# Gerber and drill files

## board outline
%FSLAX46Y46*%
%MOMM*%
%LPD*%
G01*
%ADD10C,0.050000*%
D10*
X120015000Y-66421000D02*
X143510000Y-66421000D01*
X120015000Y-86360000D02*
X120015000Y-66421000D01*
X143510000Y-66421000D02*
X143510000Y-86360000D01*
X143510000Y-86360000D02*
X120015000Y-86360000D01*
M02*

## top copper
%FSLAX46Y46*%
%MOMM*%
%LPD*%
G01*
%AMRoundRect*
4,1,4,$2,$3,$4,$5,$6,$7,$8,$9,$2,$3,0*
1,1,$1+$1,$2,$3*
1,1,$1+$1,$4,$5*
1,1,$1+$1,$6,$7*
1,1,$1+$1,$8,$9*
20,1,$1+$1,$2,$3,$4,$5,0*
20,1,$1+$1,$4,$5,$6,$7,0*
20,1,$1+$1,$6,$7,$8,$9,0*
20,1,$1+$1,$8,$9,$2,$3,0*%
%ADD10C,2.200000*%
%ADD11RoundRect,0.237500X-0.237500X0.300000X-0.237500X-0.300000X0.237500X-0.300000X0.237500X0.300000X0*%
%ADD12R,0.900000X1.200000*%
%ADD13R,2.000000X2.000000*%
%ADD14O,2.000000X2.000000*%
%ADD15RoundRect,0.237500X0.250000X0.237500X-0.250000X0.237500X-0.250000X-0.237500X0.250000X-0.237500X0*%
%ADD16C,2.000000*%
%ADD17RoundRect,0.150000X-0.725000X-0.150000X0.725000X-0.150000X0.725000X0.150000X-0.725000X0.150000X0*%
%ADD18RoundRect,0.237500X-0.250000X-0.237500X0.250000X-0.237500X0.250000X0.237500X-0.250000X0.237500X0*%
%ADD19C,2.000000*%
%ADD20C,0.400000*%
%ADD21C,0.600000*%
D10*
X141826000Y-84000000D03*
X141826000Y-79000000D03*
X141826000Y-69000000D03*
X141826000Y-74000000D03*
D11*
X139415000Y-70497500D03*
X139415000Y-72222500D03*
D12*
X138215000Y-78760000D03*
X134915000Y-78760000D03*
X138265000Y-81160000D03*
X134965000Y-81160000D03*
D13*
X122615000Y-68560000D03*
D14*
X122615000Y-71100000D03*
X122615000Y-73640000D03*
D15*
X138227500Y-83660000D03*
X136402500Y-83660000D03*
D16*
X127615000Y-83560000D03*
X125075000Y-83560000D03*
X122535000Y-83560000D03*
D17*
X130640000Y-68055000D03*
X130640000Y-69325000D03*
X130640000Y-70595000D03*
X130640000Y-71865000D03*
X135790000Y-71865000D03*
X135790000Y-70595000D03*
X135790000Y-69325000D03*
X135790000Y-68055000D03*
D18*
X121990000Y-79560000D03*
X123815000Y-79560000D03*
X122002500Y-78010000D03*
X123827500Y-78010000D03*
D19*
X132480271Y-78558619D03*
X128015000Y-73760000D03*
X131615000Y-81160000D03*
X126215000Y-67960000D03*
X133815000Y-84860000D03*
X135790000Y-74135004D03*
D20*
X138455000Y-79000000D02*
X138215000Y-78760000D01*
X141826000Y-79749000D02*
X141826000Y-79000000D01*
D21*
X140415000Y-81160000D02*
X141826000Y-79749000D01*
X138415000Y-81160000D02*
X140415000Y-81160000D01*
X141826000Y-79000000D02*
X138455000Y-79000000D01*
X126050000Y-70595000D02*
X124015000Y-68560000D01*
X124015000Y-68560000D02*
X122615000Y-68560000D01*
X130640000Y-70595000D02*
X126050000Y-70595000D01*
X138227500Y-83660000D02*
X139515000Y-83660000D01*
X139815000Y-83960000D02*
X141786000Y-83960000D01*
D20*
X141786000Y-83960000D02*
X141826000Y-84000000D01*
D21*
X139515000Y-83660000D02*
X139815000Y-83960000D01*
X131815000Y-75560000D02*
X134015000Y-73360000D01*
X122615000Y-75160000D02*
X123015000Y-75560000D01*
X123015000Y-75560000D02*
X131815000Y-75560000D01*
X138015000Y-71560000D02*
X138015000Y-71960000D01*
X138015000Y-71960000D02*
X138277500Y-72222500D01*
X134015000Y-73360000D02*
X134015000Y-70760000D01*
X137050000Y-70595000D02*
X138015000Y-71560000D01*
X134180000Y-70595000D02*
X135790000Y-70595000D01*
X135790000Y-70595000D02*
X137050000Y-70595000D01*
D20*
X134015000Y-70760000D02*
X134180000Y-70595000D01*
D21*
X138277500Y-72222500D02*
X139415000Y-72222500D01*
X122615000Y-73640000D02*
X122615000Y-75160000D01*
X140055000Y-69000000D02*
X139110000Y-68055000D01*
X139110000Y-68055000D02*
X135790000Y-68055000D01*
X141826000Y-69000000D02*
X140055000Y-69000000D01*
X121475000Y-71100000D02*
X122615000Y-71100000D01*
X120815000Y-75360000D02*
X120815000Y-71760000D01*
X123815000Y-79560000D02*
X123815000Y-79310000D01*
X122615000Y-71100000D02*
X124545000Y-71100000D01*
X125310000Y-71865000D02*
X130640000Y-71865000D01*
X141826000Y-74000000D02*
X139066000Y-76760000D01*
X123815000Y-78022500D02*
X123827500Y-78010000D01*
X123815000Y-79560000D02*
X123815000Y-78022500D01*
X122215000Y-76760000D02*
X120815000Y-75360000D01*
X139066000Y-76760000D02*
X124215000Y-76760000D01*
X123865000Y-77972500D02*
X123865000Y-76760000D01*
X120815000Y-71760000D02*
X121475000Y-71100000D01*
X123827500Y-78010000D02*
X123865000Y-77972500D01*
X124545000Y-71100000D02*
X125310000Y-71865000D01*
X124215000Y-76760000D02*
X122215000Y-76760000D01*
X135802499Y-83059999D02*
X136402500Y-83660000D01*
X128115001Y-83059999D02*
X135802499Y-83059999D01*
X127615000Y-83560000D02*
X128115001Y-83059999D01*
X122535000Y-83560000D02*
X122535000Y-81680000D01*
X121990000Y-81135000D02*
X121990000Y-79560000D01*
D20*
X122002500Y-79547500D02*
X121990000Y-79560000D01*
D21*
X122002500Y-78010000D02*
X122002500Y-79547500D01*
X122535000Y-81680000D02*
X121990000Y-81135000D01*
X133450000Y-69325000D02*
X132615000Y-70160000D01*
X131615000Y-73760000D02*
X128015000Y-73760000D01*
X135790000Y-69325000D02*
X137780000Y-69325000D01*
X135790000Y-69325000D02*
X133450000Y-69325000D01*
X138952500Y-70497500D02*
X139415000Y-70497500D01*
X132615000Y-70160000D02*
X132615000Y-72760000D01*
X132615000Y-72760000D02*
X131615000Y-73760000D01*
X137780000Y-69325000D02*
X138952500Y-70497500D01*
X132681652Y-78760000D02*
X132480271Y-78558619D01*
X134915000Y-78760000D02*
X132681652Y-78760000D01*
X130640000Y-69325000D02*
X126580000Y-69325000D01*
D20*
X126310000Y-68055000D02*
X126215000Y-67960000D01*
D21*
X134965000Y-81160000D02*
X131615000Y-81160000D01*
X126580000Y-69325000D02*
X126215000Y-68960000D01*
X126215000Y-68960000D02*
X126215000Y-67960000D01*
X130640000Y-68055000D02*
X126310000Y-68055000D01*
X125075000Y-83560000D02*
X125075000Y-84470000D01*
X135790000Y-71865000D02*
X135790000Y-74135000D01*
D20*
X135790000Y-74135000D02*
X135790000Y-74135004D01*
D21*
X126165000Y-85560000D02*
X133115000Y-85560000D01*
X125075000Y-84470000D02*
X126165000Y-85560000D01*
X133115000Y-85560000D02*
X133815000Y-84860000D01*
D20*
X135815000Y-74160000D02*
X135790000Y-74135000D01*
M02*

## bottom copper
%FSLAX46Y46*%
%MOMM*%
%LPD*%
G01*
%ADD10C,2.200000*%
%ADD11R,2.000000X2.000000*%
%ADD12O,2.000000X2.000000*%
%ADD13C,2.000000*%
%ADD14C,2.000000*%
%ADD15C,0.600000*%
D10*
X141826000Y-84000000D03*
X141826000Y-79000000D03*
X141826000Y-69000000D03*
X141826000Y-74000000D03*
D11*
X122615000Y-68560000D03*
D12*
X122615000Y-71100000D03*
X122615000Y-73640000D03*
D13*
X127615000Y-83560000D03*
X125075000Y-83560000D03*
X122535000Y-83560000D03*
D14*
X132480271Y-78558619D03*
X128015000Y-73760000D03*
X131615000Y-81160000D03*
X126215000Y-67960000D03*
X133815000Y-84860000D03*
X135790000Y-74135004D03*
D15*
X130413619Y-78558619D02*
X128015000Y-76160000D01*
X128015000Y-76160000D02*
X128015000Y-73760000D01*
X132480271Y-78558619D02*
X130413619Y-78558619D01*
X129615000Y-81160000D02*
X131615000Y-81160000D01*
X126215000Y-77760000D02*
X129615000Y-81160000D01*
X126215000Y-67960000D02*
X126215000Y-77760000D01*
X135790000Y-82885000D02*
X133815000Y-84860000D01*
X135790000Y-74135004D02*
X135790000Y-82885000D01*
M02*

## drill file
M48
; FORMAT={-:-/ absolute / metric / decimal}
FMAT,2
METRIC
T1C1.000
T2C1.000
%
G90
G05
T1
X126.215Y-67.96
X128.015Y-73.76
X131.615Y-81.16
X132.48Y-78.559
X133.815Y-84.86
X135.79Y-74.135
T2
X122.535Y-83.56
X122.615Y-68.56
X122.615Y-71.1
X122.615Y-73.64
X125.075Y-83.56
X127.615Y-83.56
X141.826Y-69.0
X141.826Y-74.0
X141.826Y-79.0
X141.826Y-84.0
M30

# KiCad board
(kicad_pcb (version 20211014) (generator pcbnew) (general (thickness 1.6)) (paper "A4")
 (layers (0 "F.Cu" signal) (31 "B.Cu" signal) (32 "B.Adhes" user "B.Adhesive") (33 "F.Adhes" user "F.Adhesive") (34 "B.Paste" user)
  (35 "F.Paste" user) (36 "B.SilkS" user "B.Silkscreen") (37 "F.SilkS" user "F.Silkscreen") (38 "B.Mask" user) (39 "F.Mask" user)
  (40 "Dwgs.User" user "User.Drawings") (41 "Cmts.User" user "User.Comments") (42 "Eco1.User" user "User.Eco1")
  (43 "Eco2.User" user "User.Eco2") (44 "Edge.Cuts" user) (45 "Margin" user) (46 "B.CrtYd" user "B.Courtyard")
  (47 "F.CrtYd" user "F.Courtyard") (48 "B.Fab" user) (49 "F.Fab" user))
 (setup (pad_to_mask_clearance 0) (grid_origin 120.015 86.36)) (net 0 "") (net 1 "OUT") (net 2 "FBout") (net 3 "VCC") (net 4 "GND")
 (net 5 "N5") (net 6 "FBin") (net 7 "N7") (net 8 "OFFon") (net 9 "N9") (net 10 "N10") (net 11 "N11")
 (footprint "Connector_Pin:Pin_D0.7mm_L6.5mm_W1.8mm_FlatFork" (layer "F.Cu") (at 141.826 84)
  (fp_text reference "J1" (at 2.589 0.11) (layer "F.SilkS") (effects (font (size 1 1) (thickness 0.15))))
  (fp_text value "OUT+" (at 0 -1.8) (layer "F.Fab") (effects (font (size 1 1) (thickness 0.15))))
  (pad "1" thru_hole circle locked (at 0 0) (size 2.2 2.2) (drill 1) (layers *.Cu *.Mask) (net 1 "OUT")))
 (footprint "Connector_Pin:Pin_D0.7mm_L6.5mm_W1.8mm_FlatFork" (layer "F.Cu") (at 141.826 79)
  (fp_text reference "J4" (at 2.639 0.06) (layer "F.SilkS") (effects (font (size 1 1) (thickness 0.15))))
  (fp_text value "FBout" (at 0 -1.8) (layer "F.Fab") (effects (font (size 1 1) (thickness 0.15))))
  (pad "1" thru_hole circle locked (at 0 0) (size 2.2 2.2) (drill 1) (layers *.Cu *.Mask) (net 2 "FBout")))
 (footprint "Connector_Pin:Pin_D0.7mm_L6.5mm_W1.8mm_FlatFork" (layer "F.Cu") (at 141.826 69)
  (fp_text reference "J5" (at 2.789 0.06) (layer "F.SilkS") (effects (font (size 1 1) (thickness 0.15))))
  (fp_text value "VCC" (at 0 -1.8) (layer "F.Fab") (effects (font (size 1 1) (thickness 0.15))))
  (pad "1" thru_hole circle locked (at 0 0) (size 2.2 2.2) (drill 1) (layers *.Cu *.Mask) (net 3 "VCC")))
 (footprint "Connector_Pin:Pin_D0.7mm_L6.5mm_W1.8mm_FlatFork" (layer "F.Cu") (at 141.826 74)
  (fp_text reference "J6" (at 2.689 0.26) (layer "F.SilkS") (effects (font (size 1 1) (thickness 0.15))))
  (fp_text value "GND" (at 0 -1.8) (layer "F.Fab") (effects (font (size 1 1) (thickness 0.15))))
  (pad "1" thru_hole circle locked (at 0 0) (size 2.2 2.2) (drill 1) (layers *.Cu *.Mask) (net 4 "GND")))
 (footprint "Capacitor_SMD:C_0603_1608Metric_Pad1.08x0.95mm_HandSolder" (layer "F.Cu") (at 139.415 71.36 -90)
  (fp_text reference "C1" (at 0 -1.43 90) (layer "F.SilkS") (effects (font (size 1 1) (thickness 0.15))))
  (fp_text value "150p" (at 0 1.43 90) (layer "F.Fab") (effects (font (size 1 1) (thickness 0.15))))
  (pad "1" smd roundrect locked (at -0.8625 0 270) (size 1.075 0.95) (layers "F.Cu" "F.Paste" "F.Mask") (roundrect_rratio 0.25) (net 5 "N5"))
  (pad "2" smd roundrect locked (at 0.8625 0 270) (size 1.075 0.95) (layers "F.Cu" "F.Paste" "F.Mask") (roundrect_rratio 0.25)
   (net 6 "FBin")))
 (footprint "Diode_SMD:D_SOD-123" (layer "F.Cu") (at 136.565 78.76 180)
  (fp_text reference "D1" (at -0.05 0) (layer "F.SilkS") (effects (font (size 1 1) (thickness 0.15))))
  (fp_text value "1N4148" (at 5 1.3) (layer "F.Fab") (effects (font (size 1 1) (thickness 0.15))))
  (pad "1" smd rect locked (at -1.65 0 180) (size 0.9 1.2) (layers "F.Cu" "F.Paste" "F.Mask") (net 2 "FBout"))
  (pad "2" smd rect locked (at 1.65 0 180) (size 0.9 1.2) (layers "F.Cu" "F.Paste" "F.Mask") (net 5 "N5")))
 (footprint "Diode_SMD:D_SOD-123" (layer "F.Cu") (at 136.615 81.16 180)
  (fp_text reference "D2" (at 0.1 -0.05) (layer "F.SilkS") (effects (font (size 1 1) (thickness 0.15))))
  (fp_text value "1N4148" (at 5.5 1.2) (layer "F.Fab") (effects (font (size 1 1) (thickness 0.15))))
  (pad "1" smd rect locked (at -1.65 0 180) (size 0.9 1.2) (layers "F.Cu" "F.Paste" "F.Mask") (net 2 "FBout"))
  (pad "2" smd rect locked (at 1.65 0 180) (size 0.9 1.2) (layers "F.Cu" "F.Paste" "F.Mask") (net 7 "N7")))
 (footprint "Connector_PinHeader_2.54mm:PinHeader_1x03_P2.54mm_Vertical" (layer "F.Cu") (at 122.615 68.56)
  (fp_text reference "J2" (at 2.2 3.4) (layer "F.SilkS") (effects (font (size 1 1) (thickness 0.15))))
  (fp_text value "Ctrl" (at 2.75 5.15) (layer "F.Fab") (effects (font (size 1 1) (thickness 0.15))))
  (pad "1" thru_hole rect locked (at 0 0) (size 2 2) (drill 1) (layers *.Cu *.Mask) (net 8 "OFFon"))
  (pad "2" thru_hole oval locked (at 0 2.54) (size 2 2) (drill 1) (layers *.Cu *.Mask) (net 4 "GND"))
  (pad "3" thru_hole oval locked (at 0 5.08) (size 2 2) (drill 1) (layers *.Cu *.Mask) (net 6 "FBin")))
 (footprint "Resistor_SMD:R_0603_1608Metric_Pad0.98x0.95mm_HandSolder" (layer "F.Cu") (at 137.315 83.66 180)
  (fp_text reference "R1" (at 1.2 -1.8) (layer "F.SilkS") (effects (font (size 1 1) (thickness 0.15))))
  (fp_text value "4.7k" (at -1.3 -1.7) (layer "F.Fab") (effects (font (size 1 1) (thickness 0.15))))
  (pad "1" smd roundrect locked (at -0.9125 0 180) (size 0.975 0.95) (layers "F.Cu" "F.Paste" "F.Mask") (roundrect_rratio 0.25)
   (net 1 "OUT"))
  (pad "2" smd roundrect locked (at 0.9125 0 180) (size 0.975 0.95) (layers "F.Cu" "F.Paste" "F.Mask") (roundrect_rratio 0.25) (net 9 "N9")))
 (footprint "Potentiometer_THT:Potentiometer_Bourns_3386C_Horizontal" (layer "F.Cu") (at 127.615 83.56 -90)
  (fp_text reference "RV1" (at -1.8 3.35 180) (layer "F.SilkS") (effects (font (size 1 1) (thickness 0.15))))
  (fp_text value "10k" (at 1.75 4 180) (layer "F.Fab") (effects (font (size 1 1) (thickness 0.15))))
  (pad "1" thru_hole circle locked (at 0 0 270) (size 2 2) (drill 1) (layers *.Cu *.Mask) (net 9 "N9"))
  (pad "2" thru_hole circle locked (at 0 2.54 270) (size 2 2) (drill 1) (layers *.Cu *.Mask) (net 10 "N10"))
  (pad "3" thru_hole circle locked (at 0 5.08 270) (size 2 2) (drill 1) (layers *.Cu *.Mask) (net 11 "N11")))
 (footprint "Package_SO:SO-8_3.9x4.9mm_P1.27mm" (layer "F.Cu") (at 133.215 69.96)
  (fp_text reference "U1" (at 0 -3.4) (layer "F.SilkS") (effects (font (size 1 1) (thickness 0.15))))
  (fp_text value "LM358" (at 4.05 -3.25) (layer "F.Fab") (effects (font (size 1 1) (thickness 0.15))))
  (pad "1" smd roundrect locked (at -2.575 -1.905) (size 1.75 0.6) (layers "F.Cu" "F.Paste" "F.Mask") (roundrect_rratio 0.25) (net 7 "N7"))
  (pad "2" smd roundrect locked (at -2.575 -0.635) (size 1.75 0.6) (layers "F.Cu" "F.Paste" "F.Mask") (roundrect_rratio 0.25) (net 7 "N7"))
  (pad "3" smd roundrect locked (at -2.575 0.635) (size 1.75 0.6) (layers "F.Cu" "F.Paste" "F.Mask") (roundrect_rratio 0.25) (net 8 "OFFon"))
  (pad "4" smd roundrect locked (at -2.575 1.905) (size 1.75 0.6) (layers "F.Cu" "F.Paste" "F.Mask") (roundrect_rratio 0.25) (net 4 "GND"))
  (pad "5" smd roundrect locked (at 2.575 1.905) (size 1.75 0.6) (layers "F.Cu" "F.Paste" "F.Mask") (roundrect_rratio 0.25) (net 10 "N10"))
  (pad "6" smd roundrect locked (at 2.575 0.635) (size 1.75 0.6) (layers "F.Cu" "F.Paste" "F.Mask") (roundrect_rratio 0.25) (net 6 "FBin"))
  (pad "7" smd roundrect locked (at 2.575 -0.635) (size 1.75 0.6) (layers "F.Cu" "F.Paste" "F.Mask") (roundrect_rratio 0.25) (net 5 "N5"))
  (pad "8" smd roundrect locked (at 2.575 -1.905) (size 1.75 0.6) (layers "F.Cu" "F.Paste" "F.Mask") (roundrect_rratio 0.25) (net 3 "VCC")))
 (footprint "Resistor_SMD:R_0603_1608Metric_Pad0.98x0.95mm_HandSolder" (layer "F.Cu") (at 122.9025 79.56)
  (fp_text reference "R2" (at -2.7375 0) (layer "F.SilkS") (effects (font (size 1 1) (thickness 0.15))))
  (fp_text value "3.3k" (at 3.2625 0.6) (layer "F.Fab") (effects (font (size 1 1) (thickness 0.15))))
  (pad "1" smd roundrect locked (at -0.9125 0) (size 0.975 0.95) (layers "F.Cu" "F.Paste" "F.Mask") (roundrect_rratio 0.25) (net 11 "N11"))
  (pad "2" smd roundrect locked (at 0.9125 0) (size 0.975 0.95) (layers "F.Cu" "F.Paste" "F.Mask") (roundrect_rratio 0.25) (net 4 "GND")))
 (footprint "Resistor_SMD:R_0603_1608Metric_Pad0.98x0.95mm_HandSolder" (layer "F.Cu") (at 122.915 78.01)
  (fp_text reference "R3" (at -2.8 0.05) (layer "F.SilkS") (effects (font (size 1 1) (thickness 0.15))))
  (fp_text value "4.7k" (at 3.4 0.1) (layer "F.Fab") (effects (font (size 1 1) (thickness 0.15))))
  (pad "1" smd roundrect locked (at -0.9125 0) (size 0.975 0.95) (layers "F.Cu" "F.Paste" "F.Mask") (roundrect_rratio 0.25) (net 11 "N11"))
  (pad "2" smd roundrect locked (at 0.9125 0) (size 0.975 0.95) (layers "F.Cu" "F.Paste" "F.Mask") (roundrect_rratio 0.25) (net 4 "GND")))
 (gr_line (start 120.015 66.421) (end 143.51 66.421) (layer "Edge.Cuts") (width 0.05))
 (gr_line (start 120.015 86.36) (end 120.015 66.421) (layer "Edge.Cuts") (width 0.05))
 (gr_line (start 143.51 66.421) (end 143.51 86.36) (layer "Edge.Cuts") (width 0.05))
 (gr_line (start 143.51 86.36) (end 120.015 86.36) (layer "Edge.Cuts") (width 0.05))
 (segment (start 138.455 79) (end 138.215 78.76) (width 0.4) (layer "F.Cu") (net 2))
 (segment (start 141.826 79.749) (end 141.826 79) (width 0.4) (layer "F.Cu") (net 2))
 (segment (start 140.415 81.16) (end 141.826 79.749) (width 0.6) (layer "F.Cu") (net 2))
 (segment (start 138.415 81.16) (end 140.415 81.16) (width 0.6) (layer "F.Cu") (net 2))
 (segment (start 141.826 79) (end 138.455 79) (width 0.6) (layer "F.Cu") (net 2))
 (segment (start 126.05 70.595) (end 124.015 68.56) (width 0.6) (layer "F.Cu") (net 8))
 (segment (start 124.015 68.56) (end 122.615 68.56) (width 0.6) (layer "F.Cu") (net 8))
 (segment (start 130.64 70.595) (end 126.05 70.595) (width 0.6) (layer "F.Cu") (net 8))
 (segment (start 138.2275 83.66) (end 139.515 83.66) (width 0.6) (layer "F.Cu") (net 1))
 (segment (start 139.815 83.96) (end 141.786 83.96) (width 0.6) (layer "F.Cu") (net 1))
 (segment (start 141.786 83.96) (end 141.826 84) (width 0.4) (layer "F.Cu") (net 1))
 (segment (start 139.515 83.66) (end 139.815 83.96) (width 0.6) (layer "F.Cu") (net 1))
 (segment (start 131.815 75.56) (end 134.015 73.36) (width 0.6) (layer "F.Cu") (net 6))
 (segment (start 122.615 75.16) (end 123.015 75.56) (width 0.6) (layer "F.Cu") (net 6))
 (segment (start 123.015 75.56) (end 131.815 75.56) (width 0.6) (layer "F.Cu") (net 6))
 (segment (start 138.015 71.56) (end 138.015 71.96) (width 0.6) (layer "F.Cu") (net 6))
 (segment (start 138.015 71.96) (end 138.2775 72.2225) (width 0.6) (layer "F.Cu") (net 6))
 (segment (start 134.015 73.36) (end 134.015 70.76) (width 0.6) (layer "F.Cu") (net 6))
 (segment (start 137.05 70.595) (end 138.015 71.56) (width 0.6) (layer "F.Cu") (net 6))
 (segment (start 134.18 70.595) (end 135.79 70.595) (width 0.6) (layer "F.Cu") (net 6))
 (segment (start 135.79 70.595) (end 137.05 70.595) (width 0.6) (layer "F.Cu") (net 6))
 (segment (start 134.015 70.76) (end 134.18 70.595) (width 0.4) (layer "F.Cu") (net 6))
 (segment (start 138.2775 72.2225) (end 139.415 72.2225) (width 0.6) (layer "F.Cu") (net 6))
 (segment (start 122.615 73.64) (end 122.615 75.16) (width 0.6) (layer "F.Cu") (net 6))
 (segment (start 140.055 69) (end 139.11 68.055) (width 0.6) (layer "F.Cu") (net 3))
 (segment (start 139.11 68.055) (end 135.79 68.055) (width 0.6) (layer "F.Cu") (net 3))
 (segment (start 141.826 69) (end 140.055 69) (width 0.6) (layer "F.Cu") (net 3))
 (segment (start 121.475 71.1) (end 122.615 71.1) (width 0.6) (layer "F.Cu") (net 4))
 (segment (start 120.815 75.36) (end 120.815 71.76) (width 0.6) (layer "F.Cu") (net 4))
 (segment (start 123.815 79.56) (end 123.815 79.31) (width 0.6) (layer "F.Cu") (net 4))
 (segment (start 122.615 71.1) (end 124.545 71.1) (width 0.6) (layer "F.Cu") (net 4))
 (segment (start 125.31 71.865) (end 130.64 71.865) (width 0.6) (layer "F.Cu") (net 4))
 (segment (start 141.826 74) (end 139.066 76.76) (width 0.6) (layer "F.Cu") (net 4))
 (segment (start 123.815 78.0225) (end 123.8275 78.01) (width 0.6) (layer "F.Cu") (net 4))
 (segment (start 123.815 79.56) (end 123.815 78.0225) (width 0.6) (layer "F.Cu") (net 4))
 (segment (start 122.215 76.76) (end 120.815 75.36) (width 0.6) (layer "F.Cu") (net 4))
 (segment (start 139.066 76.76) (end 124.215 76.76) (width 0.6) (layer "F.Cu") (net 4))
 (segment (start 123.865 77.9725) (end 123.865 76.76) (width 0.6) (layer "F.Cu") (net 4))
 (segment (start 120.815 71.76) (end 121.475 71.1) (width 0.6) (layer "F.Cu") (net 4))
 (segment (start 123.8275 78.01) (end 123.865 77.9725) (width 0.6) (layer "F.Cu") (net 4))
 (segment (start 124.545 71.1) (end 125.31 71.865) (width 0.6) (layer "F.Cu") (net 4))
 (segment (start 124.215 76.76) (end 122.215 76.76) (width 0.6) (layer "F.Cu") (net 4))
 (segment (start 135.802499 83.059999) (end 136.4025 83.66) (width 0.6) (layer "F.Cu") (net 9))
 (segment (start 128.115001 83.059999) (end 135.802499 83.059999) (width 0.6) (layer "F.Cu") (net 9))
 (segment (start 127.615 83.56) (end 128.115001 83.059999) (width 0.6) (layer "F.Cu") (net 9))
 (segment (start 122.535 83.56) (end 122.535 81.68) (width 0.6) (layer "F.Cu") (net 11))
 (segment (start 121.99 81.135) (end 121.99 79.56) (width 0.6) (layer "F.Cu") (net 11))
 (segment (start 122.0025 79.5475) (end 121.99 79.56) (width 0.4) (layer "F.Cu") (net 11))
 (segment (start 122.0025 78.01) (end 122.0025 79.5475) (width 0.6) (layer "F.Cu") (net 11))
 (segment (start 122.535 81.68) (end 121.99 81.135) (width 0.6) (layer "F.Cu") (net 11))
 (segment (start 133.45 69.325) (end 132.615 70.16) (width 0.6) (layer "F.Cu") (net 5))
 (segment (start 131.615 73.76) (end 128.015 73.76) (width 0.6) (layer "F.Cu") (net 5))
 (segment (start 135.79 69.325) (end 137.78 69.325) (width 0.6) (layer "F.Cu") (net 5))
 (segment (start 135.79 69.325) (end 133.45 69.325) (width 0.6) (layer "F.Cu") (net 5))
 (segment (start 138.9525 70.4975) (end 139.415 70.4975) (width 0.6) (layer "F.Cu") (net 5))
 (segment (start 132.615 70.16) (end 132.615 72.76) (width 0.6) (layer "F.Cu") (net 5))
 (segment (start 132.615 72.76) (end 131.615 73.76) (width 0.6) (layer "F.Cu") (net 5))
 (segment (start 137.78 69.325) (end 138.9525 70.4975) (width 0.6) (layer "F.Cu") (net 5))
 (segment (start 132.681652 78.76) (end 132.480271 78.558619) (width 0.6) (layer "F.Cu") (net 5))
 (segment (start 134.915 78.76) (end 132.681652 78.76) (width 0.6) (layer "F.Cu") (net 5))
 (via (at 132.480271 78.558619) (size 2) (drill 1) (layers "F.Cu" "B.Cu") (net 5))
 (via (at 128.015 73.76) (size 2) (drill 1) (layers "F.Cu" "B.Cu") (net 5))
 (segment (start 130.413619 78.558619) (end 128.015 76.16) (width 0.6) (layer "B.Cu") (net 5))
 (segment (start 128.015 76.16) (end 128.015 73.76) (width 0.6) (layer "B.Cu") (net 5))
 (segment (start 132.480271 78.558619) (end 130.413619 78.558619) (width 0.6) (layer "B.Cu") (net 5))
 (segment (start 130.64 69.325) (end 126.58 69.325) (width 0.6) (layer "F.Cu") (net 7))
 (segment (start 126.31 68.055) (end 126.215 67.96) (width 0.4) (layer "F.Cu") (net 7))
 (segment (start 134.965 81.16) (end 131.615 81.16) (width 0.6) (layer "F.Cu") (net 7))
 (segment (start 126.58 69.325) (end 126.215 68.96) (width 0.6) (layer "F.Cu") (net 7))
 (segment (start 126.215 68.96) (end 126.215 67.96) (width 0.6) (layer "F.Cu") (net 7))
 (segment (start 130.64 68.055) (end 126.31 68.055) (width 0.6) (layer "F.Cu") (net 7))
 (via (at 131.615 81.16) (size 2) (drill 1) (layers "F.Cu" "B.Cu") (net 7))
 (via (at 126.215 67.96) (size 2) (drill 1) (layers "F.Cu" "B.Cu") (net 7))
 (segment (start 129.615 81.16) (end 131.615 81.16) (width 0.6) (layer "B.Cu") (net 7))
 (segment (start 126.215 77.76) (end 129.615 81.16) (width 0.6) (layer "B.Cu") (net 7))
 (segment (start 126.215 67.96) (end 126.215 77.76) (width 0.6) (layer "B.Cu") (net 7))
 (segment (start 125.075 83.56) (end 125.075 84.47) (width 0.6) (layer "F.Cu") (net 10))
 (segment (start 135.79 71.865) (end 135.79 74.135) (width 0.6) (layer "F.Cu") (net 10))
 (segment (start 135.79 74.135) (end 135.79 74.135004) (width 0.4) (layer "F.Cu") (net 10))
 (segment (start 126.165 85.56) (end 133.115 85.56) (width 0.6) (layer "F.Cu") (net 10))
 (segment (start 125.075 84.47) (end 126.165 85.56) (width 0.6) (layer "F.Cu") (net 10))
 (segment (start 133.115 85.56) (end 133.815 84.86) (width 0.6) (layer "F.Cu") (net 10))
 (segment (start 135.815 74.16) (end 135.79 74.135) (width 0.4) (layer "F.Cu") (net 10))
 (via (at 133.815 84.86) (size 2) (drill 1) (layers "F.Cu" "B.Cu") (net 10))
 (via (at 135.79 74.135004) (size 2) (drill 1) (layers "F.Cu" "B.Cu") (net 10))
 (segment (start 135.79 82.885) (end 133.815 84.86) (width 0.6) (layer "B.Cu") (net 10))
 (segment (start 135.79 74.135004) (end 135.79 82.885) (width 0.6) (layer "B.Cu") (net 10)))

